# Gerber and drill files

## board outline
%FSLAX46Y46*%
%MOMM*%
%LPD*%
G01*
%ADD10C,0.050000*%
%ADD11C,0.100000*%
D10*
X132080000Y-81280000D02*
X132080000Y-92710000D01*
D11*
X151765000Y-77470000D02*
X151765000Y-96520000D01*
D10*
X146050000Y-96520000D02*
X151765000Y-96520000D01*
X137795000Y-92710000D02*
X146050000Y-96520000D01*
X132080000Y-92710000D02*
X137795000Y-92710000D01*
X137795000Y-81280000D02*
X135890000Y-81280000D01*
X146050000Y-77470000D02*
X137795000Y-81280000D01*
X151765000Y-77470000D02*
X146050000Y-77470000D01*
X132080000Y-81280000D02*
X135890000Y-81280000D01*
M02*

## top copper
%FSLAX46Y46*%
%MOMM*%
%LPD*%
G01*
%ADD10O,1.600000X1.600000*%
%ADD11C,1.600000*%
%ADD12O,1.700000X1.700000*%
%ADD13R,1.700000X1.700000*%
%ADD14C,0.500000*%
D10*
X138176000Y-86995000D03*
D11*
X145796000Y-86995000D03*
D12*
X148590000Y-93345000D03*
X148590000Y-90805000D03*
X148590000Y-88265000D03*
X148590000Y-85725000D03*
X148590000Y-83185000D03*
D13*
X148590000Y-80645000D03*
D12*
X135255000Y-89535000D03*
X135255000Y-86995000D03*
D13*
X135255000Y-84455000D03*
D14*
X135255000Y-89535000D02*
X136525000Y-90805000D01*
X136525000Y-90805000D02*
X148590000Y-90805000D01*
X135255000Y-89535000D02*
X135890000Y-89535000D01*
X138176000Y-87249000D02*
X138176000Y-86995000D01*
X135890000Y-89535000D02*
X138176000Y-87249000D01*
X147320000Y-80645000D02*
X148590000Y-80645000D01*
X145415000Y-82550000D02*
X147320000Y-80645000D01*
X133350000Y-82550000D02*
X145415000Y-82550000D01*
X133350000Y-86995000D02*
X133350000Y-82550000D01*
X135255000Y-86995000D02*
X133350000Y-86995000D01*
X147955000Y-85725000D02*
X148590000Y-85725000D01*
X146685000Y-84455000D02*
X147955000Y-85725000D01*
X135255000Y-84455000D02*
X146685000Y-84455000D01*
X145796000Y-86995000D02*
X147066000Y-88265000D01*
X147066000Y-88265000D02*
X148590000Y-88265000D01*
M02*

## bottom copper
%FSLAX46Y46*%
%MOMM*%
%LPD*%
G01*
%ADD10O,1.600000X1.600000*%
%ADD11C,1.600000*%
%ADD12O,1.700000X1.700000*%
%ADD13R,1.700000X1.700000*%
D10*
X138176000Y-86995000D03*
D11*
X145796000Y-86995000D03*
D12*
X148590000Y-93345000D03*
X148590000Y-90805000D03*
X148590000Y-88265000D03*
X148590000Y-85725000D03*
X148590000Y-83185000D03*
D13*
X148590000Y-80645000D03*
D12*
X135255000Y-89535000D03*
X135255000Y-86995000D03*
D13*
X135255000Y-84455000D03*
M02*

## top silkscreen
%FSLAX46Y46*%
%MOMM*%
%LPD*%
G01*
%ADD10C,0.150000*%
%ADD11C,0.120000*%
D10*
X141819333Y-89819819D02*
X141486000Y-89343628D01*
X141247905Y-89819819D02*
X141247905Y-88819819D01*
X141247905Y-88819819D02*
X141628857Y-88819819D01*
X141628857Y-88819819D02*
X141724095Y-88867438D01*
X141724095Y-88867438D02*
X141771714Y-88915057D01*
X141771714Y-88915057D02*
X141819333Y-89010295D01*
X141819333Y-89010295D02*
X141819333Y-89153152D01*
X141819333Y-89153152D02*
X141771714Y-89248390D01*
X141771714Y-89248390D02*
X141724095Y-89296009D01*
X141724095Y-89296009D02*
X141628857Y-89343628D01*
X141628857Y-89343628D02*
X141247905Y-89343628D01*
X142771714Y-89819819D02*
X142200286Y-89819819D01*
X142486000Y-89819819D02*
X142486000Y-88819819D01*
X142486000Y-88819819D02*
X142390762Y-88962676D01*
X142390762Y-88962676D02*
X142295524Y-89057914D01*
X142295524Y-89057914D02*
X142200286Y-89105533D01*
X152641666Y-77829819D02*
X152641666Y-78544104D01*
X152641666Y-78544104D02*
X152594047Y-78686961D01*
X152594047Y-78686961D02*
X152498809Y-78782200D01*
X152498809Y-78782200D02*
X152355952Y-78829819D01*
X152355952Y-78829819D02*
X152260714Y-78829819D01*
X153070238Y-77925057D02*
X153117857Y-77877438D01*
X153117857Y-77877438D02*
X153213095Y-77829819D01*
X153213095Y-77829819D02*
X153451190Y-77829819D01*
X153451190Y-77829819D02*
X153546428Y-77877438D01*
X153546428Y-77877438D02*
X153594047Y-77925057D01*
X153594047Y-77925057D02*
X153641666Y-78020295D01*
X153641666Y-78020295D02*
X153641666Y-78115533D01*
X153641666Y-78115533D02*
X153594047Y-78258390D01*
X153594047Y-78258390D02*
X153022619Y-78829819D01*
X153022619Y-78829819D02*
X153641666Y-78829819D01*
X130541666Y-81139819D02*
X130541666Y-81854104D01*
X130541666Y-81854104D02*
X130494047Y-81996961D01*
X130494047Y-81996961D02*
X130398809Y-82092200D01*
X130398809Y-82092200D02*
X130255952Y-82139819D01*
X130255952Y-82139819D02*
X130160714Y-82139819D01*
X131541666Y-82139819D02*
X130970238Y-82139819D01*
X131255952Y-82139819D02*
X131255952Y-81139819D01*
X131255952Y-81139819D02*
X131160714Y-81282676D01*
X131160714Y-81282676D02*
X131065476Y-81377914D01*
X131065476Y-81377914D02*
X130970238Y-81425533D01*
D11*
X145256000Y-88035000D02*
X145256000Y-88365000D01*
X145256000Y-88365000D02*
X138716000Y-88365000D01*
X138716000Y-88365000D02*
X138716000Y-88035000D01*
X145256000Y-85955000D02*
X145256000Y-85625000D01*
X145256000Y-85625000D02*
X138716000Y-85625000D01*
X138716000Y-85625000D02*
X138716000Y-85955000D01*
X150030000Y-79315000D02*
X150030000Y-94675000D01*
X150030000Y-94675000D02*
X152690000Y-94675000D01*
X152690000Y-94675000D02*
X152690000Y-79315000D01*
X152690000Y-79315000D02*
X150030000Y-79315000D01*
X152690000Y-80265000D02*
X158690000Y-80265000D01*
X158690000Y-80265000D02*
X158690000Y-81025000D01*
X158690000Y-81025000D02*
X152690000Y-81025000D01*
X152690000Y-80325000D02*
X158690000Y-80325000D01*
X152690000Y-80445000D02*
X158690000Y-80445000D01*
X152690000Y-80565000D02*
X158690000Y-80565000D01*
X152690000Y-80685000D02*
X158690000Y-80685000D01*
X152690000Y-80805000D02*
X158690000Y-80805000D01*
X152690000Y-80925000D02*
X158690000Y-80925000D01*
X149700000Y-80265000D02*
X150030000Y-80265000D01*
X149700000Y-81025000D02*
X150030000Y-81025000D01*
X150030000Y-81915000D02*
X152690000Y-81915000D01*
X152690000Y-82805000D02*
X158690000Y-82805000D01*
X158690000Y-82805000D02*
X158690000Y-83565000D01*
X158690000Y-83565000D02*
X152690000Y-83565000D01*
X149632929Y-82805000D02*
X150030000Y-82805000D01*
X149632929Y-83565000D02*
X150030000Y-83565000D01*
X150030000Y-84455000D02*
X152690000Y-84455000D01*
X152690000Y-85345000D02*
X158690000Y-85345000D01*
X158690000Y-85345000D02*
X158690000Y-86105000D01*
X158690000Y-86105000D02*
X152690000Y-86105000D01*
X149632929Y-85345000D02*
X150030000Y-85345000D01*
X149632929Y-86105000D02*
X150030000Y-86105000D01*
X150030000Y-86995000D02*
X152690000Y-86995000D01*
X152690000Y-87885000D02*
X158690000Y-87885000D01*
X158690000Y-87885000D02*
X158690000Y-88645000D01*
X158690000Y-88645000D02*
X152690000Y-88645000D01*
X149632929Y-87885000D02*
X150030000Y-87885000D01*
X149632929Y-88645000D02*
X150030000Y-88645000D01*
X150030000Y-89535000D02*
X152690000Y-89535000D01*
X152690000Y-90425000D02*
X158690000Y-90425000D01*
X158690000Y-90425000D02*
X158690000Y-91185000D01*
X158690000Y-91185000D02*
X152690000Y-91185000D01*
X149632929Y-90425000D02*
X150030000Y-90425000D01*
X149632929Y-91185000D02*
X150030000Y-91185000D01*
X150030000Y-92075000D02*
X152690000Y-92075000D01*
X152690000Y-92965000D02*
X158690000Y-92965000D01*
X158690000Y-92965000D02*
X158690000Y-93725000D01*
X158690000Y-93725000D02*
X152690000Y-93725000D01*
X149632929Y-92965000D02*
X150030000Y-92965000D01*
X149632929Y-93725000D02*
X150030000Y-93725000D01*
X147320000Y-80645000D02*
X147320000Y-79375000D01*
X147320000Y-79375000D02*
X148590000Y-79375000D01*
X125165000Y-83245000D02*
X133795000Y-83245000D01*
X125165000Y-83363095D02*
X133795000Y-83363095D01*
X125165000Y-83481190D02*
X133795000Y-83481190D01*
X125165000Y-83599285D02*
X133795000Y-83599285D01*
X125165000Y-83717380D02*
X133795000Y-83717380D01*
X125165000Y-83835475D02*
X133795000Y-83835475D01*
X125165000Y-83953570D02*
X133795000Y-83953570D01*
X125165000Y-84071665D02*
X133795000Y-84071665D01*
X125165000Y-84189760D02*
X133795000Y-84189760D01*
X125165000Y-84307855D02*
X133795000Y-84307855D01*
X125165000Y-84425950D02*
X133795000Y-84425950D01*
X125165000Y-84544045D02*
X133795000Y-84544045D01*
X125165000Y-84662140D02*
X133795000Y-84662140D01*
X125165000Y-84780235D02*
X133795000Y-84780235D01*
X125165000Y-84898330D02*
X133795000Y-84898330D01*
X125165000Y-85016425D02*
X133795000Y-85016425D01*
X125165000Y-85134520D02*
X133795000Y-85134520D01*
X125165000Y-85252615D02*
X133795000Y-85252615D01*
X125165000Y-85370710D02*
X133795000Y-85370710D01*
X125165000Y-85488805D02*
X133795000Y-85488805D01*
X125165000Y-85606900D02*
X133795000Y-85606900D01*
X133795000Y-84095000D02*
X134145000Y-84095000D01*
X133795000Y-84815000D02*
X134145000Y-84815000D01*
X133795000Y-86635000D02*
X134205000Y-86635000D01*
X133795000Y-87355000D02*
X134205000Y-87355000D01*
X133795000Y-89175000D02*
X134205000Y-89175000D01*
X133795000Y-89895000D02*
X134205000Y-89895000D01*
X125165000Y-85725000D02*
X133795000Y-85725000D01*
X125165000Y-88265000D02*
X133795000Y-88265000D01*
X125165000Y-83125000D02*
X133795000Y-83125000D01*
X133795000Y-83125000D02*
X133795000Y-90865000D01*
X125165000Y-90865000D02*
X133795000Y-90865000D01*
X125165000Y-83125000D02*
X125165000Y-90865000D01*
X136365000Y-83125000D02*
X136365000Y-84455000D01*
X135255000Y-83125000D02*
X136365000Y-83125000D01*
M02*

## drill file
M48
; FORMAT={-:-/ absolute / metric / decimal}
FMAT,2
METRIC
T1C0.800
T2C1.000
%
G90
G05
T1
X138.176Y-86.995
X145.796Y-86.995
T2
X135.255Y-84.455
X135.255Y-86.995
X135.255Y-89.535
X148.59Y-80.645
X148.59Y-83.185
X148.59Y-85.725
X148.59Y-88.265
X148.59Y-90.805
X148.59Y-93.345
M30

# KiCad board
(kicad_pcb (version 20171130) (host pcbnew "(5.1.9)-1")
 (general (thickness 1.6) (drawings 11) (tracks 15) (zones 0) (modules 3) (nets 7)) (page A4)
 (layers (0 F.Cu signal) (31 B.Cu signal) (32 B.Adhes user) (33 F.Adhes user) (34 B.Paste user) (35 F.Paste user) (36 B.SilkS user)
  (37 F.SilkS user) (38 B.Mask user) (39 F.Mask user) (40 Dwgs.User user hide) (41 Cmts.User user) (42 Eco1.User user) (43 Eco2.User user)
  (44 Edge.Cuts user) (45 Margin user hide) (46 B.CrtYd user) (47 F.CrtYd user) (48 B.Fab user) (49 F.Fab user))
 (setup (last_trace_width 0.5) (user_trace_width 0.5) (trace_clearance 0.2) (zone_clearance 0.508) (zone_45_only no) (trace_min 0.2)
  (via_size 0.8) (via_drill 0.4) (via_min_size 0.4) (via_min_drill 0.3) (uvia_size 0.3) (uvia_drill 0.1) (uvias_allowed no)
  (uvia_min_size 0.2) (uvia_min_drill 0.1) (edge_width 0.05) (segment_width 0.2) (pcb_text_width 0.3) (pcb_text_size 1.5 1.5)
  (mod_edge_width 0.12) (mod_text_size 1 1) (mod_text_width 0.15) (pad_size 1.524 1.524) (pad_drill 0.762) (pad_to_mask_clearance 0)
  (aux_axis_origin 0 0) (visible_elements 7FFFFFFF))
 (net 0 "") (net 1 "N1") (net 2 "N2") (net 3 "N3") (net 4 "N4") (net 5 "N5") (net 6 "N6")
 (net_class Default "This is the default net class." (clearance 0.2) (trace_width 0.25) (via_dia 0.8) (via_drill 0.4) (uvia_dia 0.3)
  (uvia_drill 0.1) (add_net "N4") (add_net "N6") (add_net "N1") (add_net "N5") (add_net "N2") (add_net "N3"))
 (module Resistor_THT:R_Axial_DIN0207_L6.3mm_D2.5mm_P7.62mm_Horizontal (layer F.Cu) (at 145.796 86.995 180)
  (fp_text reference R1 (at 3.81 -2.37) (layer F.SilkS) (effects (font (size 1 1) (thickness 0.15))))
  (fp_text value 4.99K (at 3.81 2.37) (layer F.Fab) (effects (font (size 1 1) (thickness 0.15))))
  (fp_line (start 0.54 -1.04) (end 0.54 -1.37) (layer F.SilkS) (width 0.12))
  (fp_line (start 0.54 -1.37) (end 7.08 -1.37) (layer F.SilkS) (width 0.12))
  (fp_line (start 7.08 -1.37) (end 7.08 -1.04) (layer F.SilkS) (width 0.12))
  (fp_line (start 0.54 1.04) (end 0.54 1.37) (layer F.SilkS) (width 0.12))
  (fp_line (start 0.54 1.37) (end 7.08 1.37) (layer F.SilkS) (width 0.12))
  (fp_line (start 7.08 1.37) (end 7.08 1.04) (layer F.SilkS) (width 0.12))
  (pad 2 thru_hole oval (at 7.62 0 180) (size 1.6 1.6) (drill 0.8) (layers *.Cu *.Mask) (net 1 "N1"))
  (pad 1 thru_hole circle (at 0 0 180) (size 1.6 1.6) (drill 0.8) (layers *.Cu *.Mask) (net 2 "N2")))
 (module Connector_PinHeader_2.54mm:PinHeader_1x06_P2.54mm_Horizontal (layer F.Cu) (at 148.59 80.645)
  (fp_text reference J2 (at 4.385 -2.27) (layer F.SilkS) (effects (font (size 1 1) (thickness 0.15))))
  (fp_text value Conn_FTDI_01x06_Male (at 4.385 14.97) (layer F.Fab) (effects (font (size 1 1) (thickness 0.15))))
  (fp_line (start 1.44 -1.33) (end 1.44 14.03) (layer F.SilkS) (width 0.12))
  (fp_line (start 1.44 14.03) (end 4.1 14.03) (layer F.SilkS) (width 0.12))
  (fp_line (start 4.1 14.03) (end 4.1 -1.33) (layer F.SilkS) (width 0.12))
  (fp_line (start 4.1 -1.33) (end 1.44 -1.33) (layer F.SilkS) (width 0.12))
  (fp_line (start 4.1 -0.38) (end 10.1 -0.38) (layer F.SilkS) (width 0.12))
  (fp_line (start 10.1 -0.38) (end 10.1 0.38) (layer F.SilkS) (width 0.12))
  (fp_line (start 10.1 0.38) (end 4.1 0.38) (layer F.SilkS) (width 0.12))
  (fp_line (start 4.1 -0.32) (end 10.1 -0.32) (layer F.SilkS) (width 0.12))
  (fp_line (start 4.1 -0.2) (end 10.1 -0.2) (layer F.SilkS) (width 0.12))
  (fp_line (start 4.1 -0.08) (end 10.1 -0.08) (layer F.SilkS) (width 0.12))
  (fp_line (start 4.1 0.04) (end 10.1 0.04) (layer F.SilkS) (width 0.12))
  (fp_line (start 4.1 0.16) (end 10.1 0.16) (layer F.SilkS) (width 0.12))
  (fp_line (start 4.1 0.28) (end 10.1 0.28) (layer F.SilkS) (width 0.12))
  (fp_line (start 1.11 -0.38) (end 1.44 -0.38) (layer F.SilkS) (width 0.12))
  (fp_line (start 1.11 0.38) (end 1.44 0.38) (layer F.SilkS) (width 0.12))
  (fp_line (start 1.44 1.27) (end 4.1 1.27) (layer F.SilkS) (width 0.12))
  (fp_line (start 4.1 2.16) (end 10.1 2.16) (layer F.SilkS) (width 0.12))
  (fp_line (start 10.1 2.16) (end 10.1 2.92) (layer F.SilkS) (width 0.12))
  (fp_line (start 10.1 2.92) (end 4.1 2.92) (layer F.SilkS) (width 0.12))
  (fp_line (start 1.042929 2.16) (end 1.44 2.16) (layer F.SilkS) (width 0.12))
  (fp_line (start 1.042929 2.92) (end 1.44 2.92) (layer F.SilkS) (width 0.12))
  (fp_line (start 1.44 3.81) (end 4.1 3.81) (layer F.SilkS) (width 0.12))
  (fp_line (start 4.1 4.7) (end 10.1 4.7) (layer F.SilkS) (width 0.12))
  (fp_line (start 10.1 4.7) (end 10.1 5.46) (layer F.SilkS) (width 0.12))
  (fp_line (start 10.1 5.46) (end 4.1 5.46) (layer F.SilkS) (width 0.12))
  (fp_line (start 1.042929 4.7) (end 1.44 4.7) (layer F.SilkS) (width 0.12))
  (fp_line (start 1.042929 5.46) (end 1.44 5.46) (layer F.SilkS) (width 0.12))
  (fp_line (start 1.44 6.35) (end 4.1 6.35) (layer F.SilkS) (width 0.12))
  (fp_line (start 4.1 7.24) (end 10.1 7.24) (layer F.SilkS) (width 0.12))
  (fp_line (start 10.1 7.24) (end 10.1 8) (layer F.SilkS) (width 0.12))
  (fp_line (start 10.1 8) (end 4.1 8) (layer F.SilkS) (width 0.12))
  (fp_line (start 1.042929 7.24) (end 1.44 7.24) (layer F.SilkS) (width 0.12))
  (fp_line (start 1.042929 8) (end 1.44 8) (layer F.SilkS) (width 0.12))
  (fp_line (start 1.44 8.89) (end 4.1 8.89) (layer F.SilkS) (width 0.12))
  (fp_line (start 4.1 9.78) (end 10.1 9.78) (layer F.SilkS) (width 0.12))
  (fp_line (start 10.1 9.78) (end 10.1 10.54) (layer F.SilkS) (width 0.12))
  (fp_line (start 10.1 10.54) (end 4.1 10.54) (layer F.SilkS) (width 0.12))
  (fp_line (start 1.042929 9.78) (end 1.44 9.78) (layer F.SilkS) (width 0.12))
  (fp_line (start 1.042929 10.54) (end 1.44 10.54) (layer F.SilkS) (width 0.12))
  (fp_line (start 1.44 11.43) (end 4.1 11.43) (layer F.SilkS) (width 0.12))
  (fp_line (start 4.1 12.32) (end 10.1 12.32) (layer F.SilkS) (width 0.12))
  (fp_line (start 10.1 12.32) (end 10.1 13.08) (layer F.SilkS) (width 0.12))
  (fp_line (start 10.1 13.08) (end 4.1 13.08) (layer F.SilkS) (width 0.12))
  (fp_line (start 1.042929 12.32) (end 1.44 12.32) (layer F.SilkS) (width 0.12))
  (fp_line (start 1.042929 13.08) (end 1.44 13.08) (layer F.SilkS) (width 0.12))
  (fp_line (start -1.27 0) (end -1.27 -1.27) (layer F.SilkS) (width 0.12))
  (fp_line (start -1.27 -1.27) (end 0 -1.27) (layer F.SilkS) (width 0.12))
  (pad 6 thru_hole oval (at 0 12.7) (size 1.7 1.7) (drill 1) (layers *.Cu *.Mask) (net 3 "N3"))
  (pad 5 thru_hole oval (at 0 10.16) (size 1.7 1.7) (drill 1) (layers *.Cu *.Mask) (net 1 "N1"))
  (pad 4 thru_hole oval (at 0 7.62) (size 1.7 1.7) (drill 1) (layers *.Cu *.Mask) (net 2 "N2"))
  (pad 3 thru_hole oval (at 0 5.08) (size 1.7 1.7) (drill 1) (layers *.Cu *.Mask) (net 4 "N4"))
  (pad 2 thru_hole oval (at 0 2.54) (size 1.7 1.7) (drill 1) (layers *.Cu *.Mask) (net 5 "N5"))
  (pad 1 thru_hole rect (at 0 0) (size 1.7 1.7) (drill 1) (layers *.Cu *.Mask) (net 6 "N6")))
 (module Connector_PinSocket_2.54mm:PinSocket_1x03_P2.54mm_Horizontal (layer F.Cu) (at 135.255 84.455)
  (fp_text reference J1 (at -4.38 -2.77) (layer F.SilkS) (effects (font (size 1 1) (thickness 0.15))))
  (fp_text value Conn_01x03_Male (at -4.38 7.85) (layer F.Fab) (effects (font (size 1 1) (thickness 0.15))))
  (fp_line (start -10.09 -1.21) (end -1.46 -1.21) (layer F.SilkS) (width 0.12))
  (fp_line (start -10.09 -1.091905) (end -1.46 -1.091905) (layer F.SilkS) (width 0.12))
  (fp_line (start -10.09 -0.97381) (end -1.46 -0.97381) (layer F.SilkS) (width 0.12))
  (fp_line (start -10.09 -0.855715) (end -1.46 -0.855715) (layer F.SilkS) (width 0.12))
  (fp_line (start -10.09 -0.73762) (end -1.46 -0.73762) (layer F.SilkS) (width 0.12))
  (fp_line (start -10.09 -0.619525) (end -1.46 -0.619525) (layer F.SilkS) (width 0.12))
  (fp_line (start -10.09 -0.50143) (end -1.46 -0.50143) (layer F.SilkS) (width 0.12))
  (fp_line (start -10.09 -0.383335) (end -1.46 -0.383335) (layer F.SilkS) (width 0.12))
  (fp_line (start -10.09 -0.26524) (end -1.46 -0.26524) (layer F.SilkS) (width 0.12))
  (fp_line (start -10.09 -0.147145) (end -1.46 -0.147145) (layer F.SilkS) (width 0.12))
  (fp_line (start -10.09 -0.02905) (end -1.46 -0.02905) (layer F.SilkS) (width 0.12))
  (fp_line (start -10.09 0.089045) (end -1.46 0.089045) (layer F.SilkS) (width 0.12))
  (fp_line (start -10.09 0.20714) (end -1.46 0.20714) (layer F.SilkS) (width 0.12))
  (fp_line (start -10.09 0.325235) (end -1.46 0.325235) (layer F.SilkS) (width 0.12))
  (fp_line (start -10.09 0.44333) (end -1.46 0.44333) (layer F.SilkS) (width 0.12))
  (fp_line (start -10.09 0.561425) (end -1.46 0.561425) (layer F.SilkS) (width 0.12))
  (fp_line (start -10.09 0.67952) (end -1.46 0.67952) (layer F.SilkS) (width 0.12))
  (fp_line (start -10.09 0.797615) (end -1.46 0.797615) (layer F.SilkS) (width 0.12))
  (fp_line (start -10.09 0.91571) (end -1.46 0.91571) (layer F.SilkS) (width 0.12))
  (fp_line (start -10.09 1.033805) (end -1.46 1.033805) (layer F.SilkS) (width 0.12))
  (fp_line (start -10.09 1.1519) (end -1.46 1.1519) (layer F.SilkS) (width 0.12))
  (fp_line (start -1.46 -0.36) (end -1.11 -0.36) (layer F.SilkS) (width 0.12))
  (fp_line (start -1.46 0.36) (end -1.11 0.36) (layer F.SilkS) (width 0.12))
  (fp_line (start -1.46 2.18) (end -1.05 2.18) (layer F.SilkS) (width 0.12))
  (fp_line (start -1.46 2.9) (end -1.05 2.9) (layer F.SilkS) (width 0.12))
  (fp_line (start -1.46 4.72) (end -1.05 4.72) (layer F.SilkS) (width 0.12))
  (fp_line (start -1.46 5.44) (end -1.05 5.44) (layer F.SilkS) (width 0.12))
  (fp_line (start -10.09 1.27) (end -1.46 1.27) (layer F.SilkS) (width 0.12))
  (fp_line (start -10.09 3.81) (end -1.46 3.81) (layer F.SilkS) (width 0.12))
  (fp_line (start -10.09 -1.33) (end -1.46 -1.33) (layer F.SilkS) (width 0.12))
  (fp_line (start -1.46 -1.33) (end -1.46 6.41) (layer F.SilkS) (width 0.12))
  (fp_line (start -10.09 6.41) (end -1.46 6.41) (layer F.SilkS) (width 0.12))
  (fp_line (start -10.09 -1.33) (end -10.09 6.41) (layer F.SilkS) (width 0.12))
  (fp_line (start 1.11 -1.33) (end 1.11 0) (layer F.SilkS) (width 0.12))
  (fp_line (start 0 -1.33) (end 1.11 -1.33) (layer F.SilkS) (width 0.12))
  (pad 3 thru_hole oval (at 0 5.08) (size 1.7 1.7) (drill 1) (layers *.Cu *.Mask) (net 1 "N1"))
  (pad 2 thru_hole oval (at 0 2.54) (size 1.7 1.7) (drill 1) (layers *.Cu *.Mask) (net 6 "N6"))
  (pad 1 thru_hole rect (at 0 0) (size 1.7 1.7) (drill 1) (layers *.Cu *.Mask) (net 4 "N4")))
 (gr_line (start 132.08 81.28) (end 132.08 92.71) (layer Edge.Cuts) (width 0.05))
 (gr_line (start 151.765 77.47) (end 151.765 96.52) (layer Edge.Cuts) (width 0.1))
 (gr_line (start 146.05 96.52) (end 151.765 96.52) (layer Edge.Cuts) (width 0.05))
 (gr_line (start 137.795 92.71) (end 146.05 96.52) (layer Edge.Cuts) (width 0.05))
 (gr_line (start 132.08 92.71) (end 137.795 92.71) (layer Edge.Cuts) (width 0.05))
 (gr_line (start 137.795 81.28) (end 135.89 81.28) (layer Edge.Cuts) (width 0.05))
 (gr_line (start 146.05 77.47) (end 137.795 81.28) (layer Edge.Cuts) (width 0.05))
 (gr_line (start 151.765 77.47) (end 146.05 77.47) (layer Edge.Cuts) (width 0.05))
 (gr_line (start 132.08 81.28) (end 135.89 81.28) (layer Edge.Cuts) (width 0.05))
 (segment (start 135.255 89.535) (end 136.525 90.805) (width 0.5) (layer F.Cu) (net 1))
 (segment (start 136.525 90.805) (end 148.59 90.805) (width 0.5) (layer F.Cu) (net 1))
 (segment (start 135.255 89.535) (end 135.89 89.535) (width 0.5) (layer F.Cu) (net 1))
 (segment (start 138.176 87.249) (end 138.176 86.995) (width 0.5) (layer F.Cu) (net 1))
 (segment (start 135.89 89.535) (end 138.176 87.249) (width 0.5) (layer F.Cu) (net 1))
 (segment (start 147.32 80.645) (end 148.59 80.645) (width 0.5) (layer F.Cu) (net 6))
 (segment (start 145.415 82.55) (end 147.32 80.645) (width 0.5) (layer F.Cu) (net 6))
 (segment (start 133.35 82.55) (end 145.415 82.55) (width 0.5) (layer F.Cu) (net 6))
 (segment (start 133.35 86.995) (end 133.35 82.55) (width 0.5) (layer F.Cu) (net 6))
 (segment (start 135.255 86.995) (end 133.35 86.995) (width 0.5) (layer F.Cu) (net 6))
 (segment (start 147.955 85.725) (end 148.59 85.725) (width 0.5) (layer F.Cu) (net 4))
 (segment (start 146.685 84.455) (end 147.955 85.725) (width 0.5) (layer F.Cu) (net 4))
 (segment (start 135.255 84.455) (end 146.685 84.455) (width 0.5) (layer F.Cu) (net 4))
 (segment (start 145.796 86.995) (end 147.066 88.265) (width 0.5) (layer F.Cu) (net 2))
 (segment (start 147.066 88.265) (end 148.59 88.265) (width 0.5) (layer F.Cu) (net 2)))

